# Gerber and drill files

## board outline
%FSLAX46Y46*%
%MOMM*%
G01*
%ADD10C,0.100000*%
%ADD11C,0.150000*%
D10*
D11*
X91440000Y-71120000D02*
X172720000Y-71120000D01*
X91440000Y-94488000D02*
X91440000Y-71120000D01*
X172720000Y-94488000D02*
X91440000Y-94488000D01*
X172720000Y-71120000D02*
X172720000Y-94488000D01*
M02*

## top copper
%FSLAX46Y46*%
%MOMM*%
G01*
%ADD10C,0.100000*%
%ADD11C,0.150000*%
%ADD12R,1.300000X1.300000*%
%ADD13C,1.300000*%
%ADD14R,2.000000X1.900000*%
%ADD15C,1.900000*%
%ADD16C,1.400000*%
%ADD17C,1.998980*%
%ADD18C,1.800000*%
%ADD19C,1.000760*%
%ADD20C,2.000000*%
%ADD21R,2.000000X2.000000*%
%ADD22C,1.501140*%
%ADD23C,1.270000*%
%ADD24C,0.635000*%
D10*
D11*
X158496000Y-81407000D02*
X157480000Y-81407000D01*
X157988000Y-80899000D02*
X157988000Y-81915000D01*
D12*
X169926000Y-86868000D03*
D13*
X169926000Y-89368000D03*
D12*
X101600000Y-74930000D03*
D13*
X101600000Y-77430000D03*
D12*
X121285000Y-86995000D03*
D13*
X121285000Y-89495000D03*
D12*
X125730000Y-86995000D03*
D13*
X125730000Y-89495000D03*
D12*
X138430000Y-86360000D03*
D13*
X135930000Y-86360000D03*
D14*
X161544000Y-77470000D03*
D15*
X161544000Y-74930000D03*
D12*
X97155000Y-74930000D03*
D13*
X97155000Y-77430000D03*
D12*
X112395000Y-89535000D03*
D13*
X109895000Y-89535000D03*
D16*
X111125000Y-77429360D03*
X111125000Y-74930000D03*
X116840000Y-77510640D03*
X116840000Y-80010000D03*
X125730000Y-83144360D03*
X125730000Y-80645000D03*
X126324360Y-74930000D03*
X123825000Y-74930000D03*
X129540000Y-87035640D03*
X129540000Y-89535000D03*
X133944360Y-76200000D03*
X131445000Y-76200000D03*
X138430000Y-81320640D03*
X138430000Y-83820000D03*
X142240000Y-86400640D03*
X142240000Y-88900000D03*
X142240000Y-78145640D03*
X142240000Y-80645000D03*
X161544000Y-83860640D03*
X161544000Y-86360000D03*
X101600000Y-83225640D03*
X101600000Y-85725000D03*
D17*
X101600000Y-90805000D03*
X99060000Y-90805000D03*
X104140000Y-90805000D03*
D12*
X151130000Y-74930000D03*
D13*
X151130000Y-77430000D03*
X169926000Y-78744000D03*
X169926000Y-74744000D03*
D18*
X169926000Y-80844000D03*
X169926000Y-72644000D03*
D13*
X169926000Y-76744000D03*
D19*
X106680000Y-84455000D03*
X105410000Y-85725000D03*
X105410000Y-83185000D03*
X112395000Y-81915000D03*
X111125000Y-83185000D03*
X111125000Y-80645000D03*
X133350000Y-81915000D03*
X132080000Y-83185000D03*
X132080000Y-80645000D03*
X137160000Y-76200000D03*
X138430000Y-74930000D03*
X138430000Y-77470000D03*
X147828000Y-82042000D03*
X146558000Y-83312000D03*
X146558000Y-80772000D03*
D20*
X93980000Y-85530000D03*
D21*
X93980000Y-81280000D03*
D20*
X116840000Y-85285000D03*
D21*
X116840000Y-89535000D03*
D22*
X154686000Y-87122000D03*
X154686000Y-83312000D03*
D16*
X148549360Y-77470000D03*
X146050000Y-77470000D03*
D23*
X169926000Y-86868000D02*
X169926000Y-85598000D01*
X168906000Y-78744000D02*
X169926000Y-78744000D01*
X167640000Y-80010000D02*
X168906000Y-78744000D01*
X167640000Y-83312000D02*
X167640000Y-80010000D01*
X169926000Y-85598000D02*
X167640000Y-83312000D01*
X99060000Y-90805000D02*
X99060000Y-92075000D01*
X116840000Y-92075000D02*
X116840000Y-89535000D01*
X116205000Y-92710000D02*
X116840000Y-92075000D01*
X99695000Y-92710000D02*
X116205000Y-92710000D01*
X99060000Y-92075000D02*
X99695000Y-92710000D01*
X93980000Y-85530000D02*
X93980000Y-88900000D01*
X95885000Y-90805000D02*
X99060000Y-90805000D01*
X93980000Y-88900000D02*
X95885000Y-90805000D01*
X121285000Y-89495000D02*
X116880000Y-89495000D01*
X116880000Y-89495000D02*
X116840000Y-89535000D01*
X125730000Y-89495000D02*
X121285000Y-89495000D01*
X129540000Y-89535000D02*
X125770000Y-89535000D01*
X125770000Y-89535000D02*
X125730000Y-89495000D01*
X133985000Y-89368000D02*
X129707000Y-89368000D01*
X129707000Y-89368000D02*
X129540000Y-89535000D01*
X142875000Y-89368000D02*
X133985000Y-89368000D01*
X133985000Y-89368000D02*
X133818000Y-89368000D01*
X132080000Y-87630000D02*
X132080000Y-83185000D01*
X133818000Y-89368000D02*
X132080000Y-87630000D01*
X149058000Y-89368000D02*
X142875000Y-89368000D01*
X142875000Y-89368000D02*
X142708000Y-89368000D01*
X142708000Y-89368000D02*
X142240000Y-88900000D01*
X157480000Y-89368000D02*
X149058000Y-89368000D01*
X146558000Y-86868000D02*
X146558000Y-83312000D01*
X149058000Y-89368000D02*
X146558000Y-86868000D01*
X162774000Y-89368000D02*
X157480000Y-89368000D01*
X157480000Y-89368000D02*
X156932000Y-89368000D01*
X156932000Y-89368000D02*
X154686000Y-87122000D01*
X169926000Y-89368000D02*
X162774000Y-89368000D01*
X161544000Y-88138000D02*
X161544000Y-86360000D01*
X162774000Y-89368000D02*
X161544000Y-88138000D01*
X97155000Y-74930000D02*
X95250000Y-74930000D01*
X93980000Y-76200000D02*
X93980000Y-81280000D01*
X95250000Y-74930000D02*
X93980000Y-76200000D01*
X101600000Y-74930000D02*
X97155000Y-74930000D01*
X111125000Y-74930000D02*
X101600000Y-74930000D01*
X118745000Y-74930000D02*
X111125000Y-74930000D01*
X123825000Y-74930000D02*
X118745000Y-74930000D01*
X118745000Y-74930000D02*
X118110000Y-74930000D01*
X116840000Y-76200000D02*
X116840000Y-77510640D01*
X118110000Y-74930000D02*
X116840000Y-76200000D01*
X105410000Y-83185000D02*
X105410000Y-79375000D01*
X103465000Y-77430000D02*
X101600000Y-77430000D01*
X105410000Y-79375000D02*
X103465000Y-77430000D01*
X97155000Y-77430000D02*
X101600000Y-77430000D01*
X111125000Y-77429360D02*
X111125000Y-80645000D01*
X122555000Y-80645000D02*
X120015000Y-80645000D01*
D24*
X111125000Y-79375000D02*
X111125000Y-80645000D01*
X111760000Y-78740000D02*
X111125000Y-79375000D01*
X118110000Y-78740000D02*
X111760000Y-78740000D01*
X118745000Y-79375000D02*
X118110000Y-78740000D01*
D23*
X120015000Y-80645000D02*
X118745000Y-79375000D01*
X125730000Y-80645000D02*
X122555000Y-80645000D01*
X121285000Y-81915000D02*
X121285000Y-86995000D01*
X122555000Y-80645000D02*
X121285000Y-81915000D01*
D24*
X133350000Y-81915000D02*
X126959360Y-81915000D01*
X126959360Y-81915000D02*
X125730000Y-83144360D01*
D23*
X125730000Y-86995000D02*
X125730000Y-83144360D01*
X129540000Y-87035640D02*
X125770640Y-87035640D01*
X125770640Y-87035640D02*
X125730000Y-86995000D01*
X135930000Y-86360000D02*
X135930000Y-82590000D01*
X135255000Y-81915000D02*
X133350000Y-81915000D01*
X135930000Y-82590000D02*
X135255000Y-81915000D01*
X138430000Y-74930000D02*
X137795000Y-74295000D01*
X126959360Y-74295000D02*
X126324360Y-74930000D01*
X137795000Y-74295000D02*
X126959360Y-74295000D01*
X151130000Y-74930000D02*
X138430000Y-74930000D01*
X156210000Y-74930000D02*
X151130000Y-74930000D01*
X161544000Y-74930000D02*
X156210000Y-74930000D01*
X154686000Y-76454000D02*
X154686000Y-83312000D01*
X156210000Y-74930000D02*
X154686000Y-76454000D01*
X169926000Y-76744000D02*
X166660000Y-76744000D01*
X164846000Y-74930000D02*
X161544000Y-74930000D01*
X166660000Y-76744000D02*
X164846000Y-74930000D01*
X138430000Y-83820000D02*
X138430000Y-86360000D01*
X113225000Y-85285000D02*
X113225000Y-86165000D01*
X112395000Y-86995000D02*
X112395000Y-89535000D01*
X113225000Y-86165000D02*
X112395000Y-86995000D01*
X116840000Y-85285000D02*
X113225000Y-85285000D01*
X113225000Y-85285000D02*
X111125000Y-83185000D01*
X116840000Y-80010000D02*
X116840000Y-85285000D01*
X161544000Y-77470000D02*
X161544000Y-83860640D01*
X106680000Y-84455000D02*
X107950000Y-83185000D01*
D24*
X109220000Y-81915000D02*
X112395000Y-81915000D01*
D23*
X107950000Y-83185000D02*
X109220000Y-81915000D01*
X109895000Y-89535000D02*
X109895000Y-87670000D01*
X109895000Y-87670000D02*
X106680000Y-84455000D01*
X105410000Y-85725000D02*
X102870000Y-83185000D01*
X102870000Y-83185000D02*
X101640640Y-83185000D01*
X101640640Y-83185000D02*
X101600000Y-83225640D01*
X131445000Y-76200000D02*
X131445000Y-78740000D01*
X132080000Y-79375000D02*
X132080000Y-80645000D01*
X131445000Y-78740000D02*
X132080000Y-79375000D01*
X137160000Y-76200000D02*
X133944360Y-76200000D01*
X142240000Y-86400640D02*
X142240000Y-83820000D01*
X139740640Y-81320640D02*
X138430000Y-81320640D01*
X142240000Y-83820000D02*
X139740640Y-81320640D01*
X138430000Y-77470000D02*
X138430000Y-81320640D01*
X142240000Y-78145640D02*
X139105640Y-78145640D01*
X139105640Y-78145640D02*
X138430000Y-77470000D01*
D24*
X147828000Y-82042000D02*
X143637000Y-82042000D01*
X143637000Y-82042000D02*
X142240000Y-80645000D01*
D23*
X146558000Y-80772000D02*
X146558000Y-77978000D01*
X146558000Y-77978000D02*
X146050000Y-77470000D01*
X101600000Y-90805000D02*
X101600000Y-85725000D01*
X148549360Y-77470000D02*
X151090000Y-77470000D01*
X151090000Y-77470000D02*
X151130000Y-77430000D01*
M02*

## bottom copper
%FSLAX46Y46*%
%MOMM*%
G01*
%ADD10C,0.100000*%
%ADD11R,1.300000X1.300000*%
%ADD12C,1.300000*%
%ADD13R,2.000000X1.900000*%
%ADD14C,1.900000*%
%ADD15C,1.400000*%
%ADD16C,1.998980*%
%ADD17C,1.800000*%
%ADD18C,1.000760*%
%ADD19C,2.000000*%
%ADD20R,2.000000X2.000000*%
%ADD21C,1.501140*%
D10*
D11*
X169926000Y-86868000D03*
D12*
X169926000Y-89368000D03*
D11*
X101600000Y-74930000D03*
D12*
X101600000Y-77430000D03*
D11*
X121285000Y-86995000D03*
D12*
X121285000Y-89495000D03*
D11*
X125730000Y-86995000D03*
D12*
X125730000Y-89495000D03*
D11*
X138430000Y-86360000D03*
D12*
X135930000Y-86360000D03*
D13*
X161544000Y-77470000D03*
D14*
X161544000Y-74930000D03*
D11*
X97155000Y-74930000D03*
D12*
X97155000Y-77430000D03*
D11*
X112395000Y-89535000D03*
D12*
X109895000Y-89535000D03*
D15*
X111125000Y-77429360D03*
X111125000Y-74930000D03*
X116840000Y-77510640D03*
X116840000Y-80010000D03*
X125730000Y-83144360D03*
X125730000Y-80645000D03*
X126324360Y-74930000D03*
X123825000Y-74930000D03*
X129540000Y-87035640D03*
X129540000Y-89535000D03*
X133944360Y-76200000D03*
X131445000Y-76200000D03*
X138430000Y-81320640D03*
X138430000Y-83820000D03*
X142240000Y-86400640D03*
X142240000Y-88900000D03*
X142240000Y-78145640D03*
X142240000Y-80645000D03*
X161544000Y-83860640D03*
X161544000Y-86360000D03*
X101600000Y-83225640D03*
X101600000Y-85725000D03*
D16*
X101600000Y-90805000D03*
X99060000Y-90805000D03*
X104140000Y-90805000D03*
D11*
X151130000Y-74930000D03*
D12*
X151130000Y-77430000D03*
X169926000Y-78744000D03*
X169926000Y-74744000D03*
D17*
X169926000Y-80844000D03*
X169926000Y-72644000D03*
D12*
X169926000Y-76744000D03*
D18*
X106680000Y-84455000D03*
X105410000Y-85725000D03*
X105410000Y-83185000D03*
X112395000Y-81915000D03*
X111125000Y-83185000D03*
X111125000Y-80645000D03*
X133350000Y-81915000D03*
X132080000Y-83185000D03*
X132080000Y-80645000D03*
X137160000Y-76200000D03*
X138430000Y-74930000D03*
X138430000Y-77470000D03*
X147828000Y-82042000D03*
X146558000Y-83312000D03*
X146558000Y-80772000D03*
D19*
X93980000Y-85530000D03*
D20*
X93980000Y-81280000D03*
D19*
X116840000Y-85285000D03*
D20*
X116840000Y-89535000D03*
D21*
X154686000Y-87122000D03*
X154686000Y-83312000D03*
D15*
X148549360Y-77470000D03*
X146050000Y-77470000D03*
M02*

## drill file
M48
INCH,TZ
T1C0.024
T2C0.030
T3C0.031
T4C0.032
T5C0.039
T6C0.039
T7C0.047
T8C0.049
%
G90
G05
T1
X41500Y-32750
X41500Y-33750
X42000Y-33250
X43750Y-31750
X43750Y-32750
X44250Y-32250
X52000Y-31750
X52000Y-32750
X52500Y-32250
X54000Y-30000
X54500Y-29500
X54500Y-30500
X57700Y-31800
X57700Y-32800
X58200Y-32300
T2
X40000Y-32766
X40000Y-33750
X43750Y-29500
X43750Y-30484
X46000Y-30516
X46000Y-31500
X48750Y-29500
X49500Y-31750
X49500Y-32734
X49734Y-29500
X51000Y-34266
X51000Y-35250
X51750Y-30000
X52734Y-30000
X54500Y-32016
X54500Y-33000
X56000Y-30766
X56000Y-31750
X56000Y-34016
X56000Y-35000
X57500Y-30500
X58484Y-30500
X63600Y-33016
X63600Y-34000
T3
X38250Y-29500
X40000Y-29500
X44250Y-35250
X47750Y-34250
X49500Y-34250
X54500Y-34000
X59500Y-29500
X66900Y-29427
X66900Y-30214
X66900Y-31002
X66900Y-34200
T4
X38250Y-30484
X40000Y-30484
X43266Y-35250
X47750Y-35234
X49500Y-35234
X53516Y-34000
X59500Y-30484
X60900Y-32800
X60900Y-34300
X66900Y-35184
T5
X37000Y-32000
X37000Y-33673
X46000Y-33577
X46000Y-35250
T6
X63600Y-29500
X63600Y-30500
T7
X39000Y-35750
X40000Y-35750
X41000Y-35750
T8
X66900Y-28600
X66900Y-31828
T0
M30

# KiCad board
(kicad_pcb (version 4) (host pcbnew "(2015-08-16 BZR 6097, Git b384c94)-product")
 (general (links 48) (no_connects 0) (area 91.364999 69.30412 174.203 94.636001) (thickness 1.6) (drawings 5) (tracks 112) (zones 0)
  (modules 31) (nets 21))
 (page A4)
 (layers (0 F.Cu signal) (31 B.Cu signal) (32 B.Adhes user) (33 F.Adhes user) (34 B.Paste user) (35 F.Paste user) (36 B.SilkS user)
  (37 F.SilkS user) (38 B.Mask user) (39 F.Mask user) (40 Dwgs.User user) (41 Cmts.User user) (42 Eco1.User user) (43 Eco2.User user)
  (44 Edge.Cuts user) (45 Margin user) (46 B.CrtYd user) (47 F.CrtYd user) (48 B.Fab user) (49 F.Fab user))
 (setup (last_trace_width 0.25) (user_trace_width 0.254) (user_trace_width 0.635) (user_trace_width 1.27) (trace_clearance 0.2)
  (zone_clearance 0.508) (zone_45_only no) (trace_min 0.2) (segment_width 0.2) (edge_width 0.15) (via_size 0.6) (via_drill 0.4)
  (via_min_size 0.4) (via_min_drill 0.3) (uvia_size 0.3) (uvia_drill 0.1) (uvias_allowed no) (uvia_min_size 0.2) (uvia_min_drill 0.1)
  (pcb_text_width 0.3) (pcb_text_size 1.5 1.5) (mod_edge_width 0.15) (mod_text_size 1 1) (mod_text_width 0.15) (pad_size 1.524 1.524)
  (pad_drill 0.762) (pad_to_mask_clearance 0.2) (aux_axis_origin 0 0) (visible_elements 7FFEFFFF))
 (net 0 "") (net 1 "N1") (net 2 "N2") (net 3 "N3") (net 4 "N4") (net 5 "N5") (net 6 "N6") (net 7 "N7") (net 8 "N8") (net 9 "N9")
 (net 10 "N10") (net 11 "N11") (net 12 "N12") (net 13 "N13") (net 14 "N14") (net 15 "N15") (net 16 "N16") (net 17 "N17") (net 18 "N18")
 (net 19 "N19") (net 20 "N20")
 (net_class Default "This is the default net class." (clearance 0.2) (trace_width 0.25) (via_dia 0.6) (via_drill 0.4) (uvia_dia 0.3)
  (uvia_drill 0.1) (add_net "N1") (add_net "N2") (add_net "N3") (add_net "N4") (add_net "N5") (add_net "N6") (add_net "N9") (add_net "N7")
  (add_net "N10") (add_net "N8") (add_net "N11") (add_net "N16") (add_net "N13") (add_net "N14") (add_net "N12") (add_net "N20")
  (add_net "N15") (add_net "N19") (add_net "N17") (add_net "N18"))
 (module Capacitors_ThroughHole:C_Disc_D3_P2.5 (layer F.Cu) (at 169.926 86.868 270)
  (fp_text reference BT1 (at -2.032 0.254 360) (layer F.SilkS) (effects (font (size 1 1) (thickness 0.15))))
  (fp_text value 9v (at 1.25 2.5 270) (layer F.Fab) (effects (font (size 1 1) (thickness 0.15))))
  (pad 1 thru_hole rect (at 0 0 270) (size 1.3 1.3) (drill 0.8) (layers *.Cu *.Mask F.SilkS) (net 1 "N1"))
  (pad 2 thru_hole circle (at 2.5 0 270) (size 1.3 1.3) (drill 0.8001) (layers *.Cu *.Mask F.SilkS) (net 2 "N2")))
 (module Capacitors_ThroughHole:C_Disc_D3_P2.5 (layer F.Cu) (at 101.6 74.93 270)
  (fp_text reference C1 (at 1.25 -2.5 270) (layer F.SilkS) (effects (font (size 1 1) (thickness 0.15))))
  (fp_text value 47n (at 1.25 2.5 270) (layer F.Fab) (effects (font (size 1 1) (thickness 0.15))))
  (pad 1 thru_hole rect (at 0 0 270) (size 1.3 1.3) (drill 0.8) (layers *.Cu *.Mask F.SilkS) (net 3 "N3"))
  (pad 2 thru_hole circle (at 2.5 0 270) (size 1.3 1.3) (drill 0.8001) (layers *.Cu *.Mask F.SilkS) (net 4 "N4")))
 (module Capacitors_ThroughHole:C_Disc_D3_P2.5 (layer F.Cu) (at 121.285 86.995 270)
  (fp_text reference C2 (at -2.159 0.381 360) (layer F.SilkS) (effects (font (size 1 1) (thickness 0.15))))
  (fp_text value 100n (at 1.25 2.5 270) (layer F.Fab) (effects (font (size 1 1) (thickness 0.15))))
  (pad 1 thru_hole rect (at 0 0 270) (size 1.3 1.3) (drill 0.8) (layers *.Cu *.Mask F.SilkS) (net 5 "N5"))
  (pad 2 thru_hole circle (at 2.5 0 270) (size 1.3 1.3) (drill 0.8001) (layers *.Cu *.Mask F.SilkS) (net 2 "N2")))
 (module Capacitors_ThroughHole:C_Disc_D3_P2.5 (layer F.Cu) (at 125.73 86.995 270)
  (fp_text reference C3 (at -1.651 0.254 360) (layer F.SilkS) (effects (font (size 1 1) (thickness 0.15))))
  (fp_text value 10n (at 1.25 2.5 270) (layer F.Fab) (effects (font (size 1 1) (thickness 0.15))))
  (pad 1 thru_hole rect (at 0 0 270) (size 1.3 1.3) (drill 0.8) (layers *.Cu *.Mask F.SilkS) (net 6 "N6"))
  (pad 2 thru_hole circle (at 2.5 0 270) (size 1.3 1.3) (drill 0.8001) (layers *.Cu *.Mask F.SilkS) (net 2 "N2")))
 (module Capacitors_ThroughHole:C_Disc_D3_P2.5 (layer F.Cu) (at 138.43 86.36 180)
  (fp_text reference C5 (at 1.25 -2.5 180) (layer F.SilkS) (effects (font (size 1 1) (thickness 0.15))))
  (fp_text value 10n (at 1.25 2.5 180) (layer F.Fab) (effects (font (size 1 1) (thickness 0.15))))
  (pad 1 thru_hole rect (at 0 0 180) (size 1.3 1.3) (drill 0.8) (layers *.Cu *.Mask F.SilkS) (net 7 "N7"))
  (pad 2 thru_hole circle (at 2.5 0 180) (size 1.3 1.3) (drill 0.8001) (layers *.Cu *.Mask F.SilkS) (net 6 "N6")))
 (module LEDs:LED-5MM (layer F.Cu) (at 161.544 77.47 90)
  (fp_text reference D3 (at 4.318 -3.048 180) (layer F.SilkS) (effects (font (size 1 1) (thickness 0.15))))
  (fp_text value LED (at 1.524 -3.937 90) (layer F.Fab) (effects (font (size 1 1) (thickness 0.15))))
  (pad 1 thru_hole rect (at 0 0 180) (size 2 1.9) (drill 1.00076) (layers *.Cu *.Mask F.SilkS) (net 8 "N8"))
  (pad 2 thru_hole circle (at 2.54 0 90) (size 1.9 1.9) (drill 1.00076) (layers *.Cu *.Mask F.SilkS) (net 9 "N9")))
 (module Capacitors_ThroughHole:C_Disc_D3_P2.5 (layer F.Cu) (at 97.155 74.93 270)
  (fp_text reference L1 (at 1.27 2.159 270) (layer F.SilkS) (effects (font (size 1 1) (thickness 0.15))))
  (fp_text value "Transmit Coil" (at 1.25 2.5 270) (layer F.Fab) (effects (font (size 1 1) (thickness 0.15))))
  (pad 1 thru_hole rect (at 0 0 270) (size 1.3 1.3) (drill 0.8) (layers *.Cu *.Mask F.SilkS) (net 3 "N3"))
  (pad 2 thru_hole circle (at 2.5 0 270) (size 1.3 1.3) (drill 0.8001) (layers *.Cu *.Mask F.SilkS) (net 4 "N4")))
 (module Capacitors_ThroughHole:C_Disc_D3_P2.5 (layer F.Cu) (at 112.395 89.535 180)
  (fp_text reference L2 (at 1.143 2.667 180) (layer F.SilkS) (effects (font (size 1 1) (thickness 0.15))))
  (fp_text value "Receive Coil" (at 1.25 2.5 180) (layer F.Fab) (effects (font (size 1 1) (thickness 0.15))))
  (pad 1 thru_hole rect (at 0 0 180) (size 1.3 1.3) (drill 0.8) (layers *.Cu *.Mask F.SilkS) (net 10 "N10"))
  (pad 2 thru_hole circle (at 2.5 0 180) (size 1.3 1.3) (drill 0.8001) (layers *.Cu *.Mask F.SilkS) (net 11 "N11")))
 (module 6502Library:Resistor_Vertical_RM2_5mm (layer F.Cu) (at 111.125 74.93 90)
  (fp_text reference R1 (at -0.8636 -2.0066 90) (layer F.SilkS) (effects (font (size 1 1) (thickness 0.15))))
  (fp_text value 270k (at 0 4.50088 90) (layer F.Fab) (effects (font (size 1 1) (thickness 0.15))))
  (pad 1 thru_hole circle (at -2.49936 0 90) (size 1.4 1.4) (drill 0.76) (layers *.Cu *.SilkS *.Mask) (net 5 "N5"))
  (pad 2 thru_hole circle (at 0 0 90) (size 1.4 1.4) (drill 0.76) (layers *.Cu *.SilkS *.Mask) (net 3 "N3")))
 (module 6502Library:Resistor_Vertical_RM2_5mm (layer F.Cu) (at 116.84 80.01 270)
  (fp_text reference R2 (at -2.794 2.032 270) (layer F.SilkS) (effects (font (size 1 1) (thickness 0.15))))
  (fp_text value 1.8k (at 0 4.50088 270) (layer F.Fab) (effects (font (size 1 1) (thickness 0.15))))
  (pad 1 thru_hole circle (at -2.49936 0 270) (size 1.4 1.4) (drill 0.76) (layers *.Cu *.SilkS *.Mask) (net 3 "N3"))
  (pad 2 thru_hole circle (at 0 0 270) (size 1.4 1.4) (drill 0.76) (layers *.Cu *.SilkS *.Mask) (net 10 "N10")))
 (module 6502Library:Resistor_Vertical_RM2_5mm (layer F.Cu) (at 125.73 80.645 90)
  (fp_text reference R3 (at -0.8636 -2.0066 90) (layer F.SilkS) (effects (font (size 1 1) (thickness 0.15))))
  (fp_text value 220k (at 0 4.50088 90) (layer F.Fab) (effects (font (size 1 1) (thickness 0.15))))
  (pad 1 thru_hole circle (at -2.49936 0 90) (size 1.4 1.4) (drill 0.76) (layers *.Cu *.SilkS *.Mask) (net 6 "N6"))
  (pad 2 thru_hole circle (at 0 0 90) (size 1.4 1.4) (drill 0.76) (layers *.Cu *.SilkS *.Mask) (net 5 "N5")))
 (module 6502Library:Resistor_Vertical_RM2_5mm (layer F.Cu) (at 123.825 74.93 180)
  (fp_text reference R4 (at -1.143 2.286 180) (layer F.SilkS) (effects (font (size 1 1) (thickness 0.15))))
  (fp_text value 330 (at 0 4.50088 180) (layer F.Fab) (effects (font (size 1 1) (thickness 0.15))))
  (pad 1 thru_hole circle (at -2.49936 0 180) (size 1.4 1.4) (drill 0.76) (layers *.Cu *.SilkS *.Mask) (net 9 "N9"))
  (pad 2 thru_hole circle (at 0 0 180) (size 1.4 1.4) (drill 0.76) (layers *.Cu *.SilkS *.Mask) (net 3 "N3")))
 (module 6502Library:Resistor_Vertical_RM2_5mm (layer F.Cu) (at 129.54 89.535 270)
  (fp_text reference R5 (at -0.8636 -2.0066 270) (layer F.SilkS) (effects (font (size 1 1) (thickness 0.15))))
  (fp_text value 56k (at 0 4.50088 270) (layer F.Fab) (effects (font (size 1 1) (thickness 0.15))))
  (pad 1 thru_hole circle (at -2.49936 0 270) (size 1.4 1.4) (drill 0.76) (layers *.Cu *.SilkS *.Mask) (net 6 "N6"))
  (pad 2 thru_hole circle (at 0 0 270) (size 1.4 1.4) (drill 0.76) (layers *.Cu *.SilkS *.Mask) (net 2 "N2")))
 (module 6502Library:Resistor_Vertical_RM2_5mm (layer F.Cu) (at 131.445 76.2 180)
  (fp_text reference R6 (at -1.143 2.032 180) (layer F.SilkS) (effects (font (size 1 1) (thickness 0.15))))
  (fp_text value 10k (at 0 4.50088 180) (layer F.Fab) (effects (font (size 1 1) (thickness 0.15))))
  (pad 1 thru_hole circle (at -2.49936 0 180) (size 1.4 1.4) (drill 0.76) (layers *.Cu *.SilkS *.Mask) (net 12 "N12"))
  (pad 2 thru_hole circle (at 0 0 180) (size 1.4 1.4) (drill 0.76) (layers *.Cu *.SilkS *.Mask) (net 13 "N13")))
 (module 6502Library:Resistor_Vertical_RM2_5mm (layer F.Cu) (at 138.43 83.82 270)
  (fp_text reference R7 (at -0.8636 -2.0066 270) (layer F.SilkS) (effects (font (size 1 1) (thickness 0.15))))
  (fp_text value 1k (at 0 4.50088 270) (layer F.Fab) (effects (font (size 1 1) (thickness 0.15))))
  (pad 1 thru_hole circle (at -2.49936 0 270) (size 1.4 1.4) (drill 0.76) (layers *.Cu *.SilkS *.Mask) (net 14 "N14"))
  (pad 2 thru_hole circle (at 0 0 270) (size 1.4 1.4) (drill 0.76) (layers *.Cu *.SilkS *.Mask) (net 7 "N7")))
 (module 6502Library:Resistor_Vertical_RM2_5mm (layer F.Cu) (at 142.24 88.9 270)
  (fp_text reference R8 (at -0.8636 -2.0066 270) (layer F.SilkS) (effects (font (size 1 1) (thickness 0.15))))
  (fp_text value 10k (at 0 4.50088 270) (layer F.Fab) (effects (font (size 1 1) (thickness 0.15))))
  (pad 1 thru_hole circle (at -2.49936 0 270) (size 1.4 1.4) (drill 0.76) (layers *.Cu *.SilkS *.Mask) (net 14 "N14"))
  (pad 2 thru_hole circle (at 0 0 270) (size 1.4 1.4) (drill 0.76) (layers *.Cu *.SilkS *.Mask) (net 2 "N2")))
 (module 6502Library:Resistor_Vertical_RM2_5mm (layer F.Cu) (at 142.24 80.645 270)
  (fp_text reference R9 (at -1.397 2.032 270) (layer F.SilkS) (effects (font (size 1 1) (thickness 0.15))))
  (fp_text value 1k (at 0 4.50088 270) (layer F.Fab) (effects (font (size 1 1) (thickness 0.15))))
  (pad 1 thru_hole circle (at -2.49936 0 270) (size 1.4 1.4) (drill 0.76) (layers *.Cu *.SilkS *.Mask) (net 14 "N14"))
  (pad 2 thru_hole circle (at 0 0 270) (size 1.4 1.4) (drill 0.76) (layers *.Cu *.SilkS *.Mask) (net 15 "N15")))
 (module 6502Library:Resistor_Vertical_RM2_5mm (layer F.Cu) (at 161.544 86.36 270)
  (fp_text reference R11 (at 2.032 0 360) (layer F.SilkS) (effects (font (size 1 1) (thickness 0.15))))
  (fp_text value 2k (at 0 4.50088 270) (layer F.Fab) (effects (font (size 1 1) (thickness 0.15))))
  (pad 1 thru_hole circle (at -2.49936 0 270) (size 1.4 1.4) (drill 0.76) (layers *.Cu *.SilkS *.Mask) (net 8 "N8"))
  (pad 2 thru_hole circle (at 0 0 270) (size 1.4 1.4) (drill 0.76) (layers *.Cu *.SilkS *.Mask) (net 2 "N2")))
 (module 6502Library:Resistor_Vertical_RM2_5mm (layer F.Cu) (at 101.6 85.725 270)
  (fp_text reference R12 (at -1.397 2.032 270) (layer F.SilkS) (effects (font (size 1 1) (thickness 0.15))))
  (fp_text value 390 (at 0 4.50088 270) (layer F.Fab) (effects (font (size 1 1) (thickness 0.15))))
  (pad 1 thru_hole circle (at -2.49936 0 270) (size 1.4 1.4) (drill 0.76) (layers *.Cu *.SilkS *.Mask) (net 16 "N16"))
  (pad 2 thru_hole circle (at 0 0 270) (size 1.4 1.4) (drill 0.76) (layers *.Cu *.SilkS *.Mask) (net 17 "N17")))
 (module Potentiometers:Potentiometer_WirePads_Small (layer F.Cu) (at 104.14 90.805 270)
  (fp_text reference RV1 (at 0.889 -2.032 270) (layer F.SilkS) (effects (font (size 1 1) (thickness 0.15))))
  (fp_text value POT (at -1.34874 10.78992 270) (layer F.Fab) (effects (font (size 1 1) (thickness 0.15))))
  (pad 2 thru_hole circle (at 0 2.54 270) (size 1.99898 1.99898) (drill 1.19888) (layers *.Cu *.Mask F.SilkS) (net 17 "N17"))
  (pad 3 thru_hole circle (at 0 5.08 270) (size 1.99898 1.99898) (drill 1.19888) (layers *.Cu *.Mask F.SilkS) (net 2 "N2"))
  (pad 1 thru_hole circle (at 0 0 270) (size 1.99898 1.99898) (drill 1.19888) (layers *.Cu *.Mask F.SilkS) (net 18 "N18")))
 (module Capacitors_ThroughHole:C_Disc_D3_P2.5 (layer F.Cu) (at 151.13 74.93 270)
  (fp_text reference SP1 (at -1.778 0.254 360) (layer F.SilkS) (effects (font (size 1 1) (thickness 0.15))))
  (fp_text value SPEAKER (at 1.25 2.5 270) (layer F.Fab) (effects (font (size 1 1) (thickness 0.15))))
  (pad 1 thru_hole rect (at 0 0 270) (size 1.3 1.3) (drill 0.8) (layers *.Cu *.Mask F.SilkS) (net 9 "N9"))
  (pad 2 thru_hole circle (at 2.5 0 270) (size 1.3 1.3) (drill 0.8001) (layers *.Cu *.Mask F.SilkS) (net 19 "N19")))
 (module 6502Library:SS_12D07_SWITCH (layer F.Cu) (at 169.926 72.644 270)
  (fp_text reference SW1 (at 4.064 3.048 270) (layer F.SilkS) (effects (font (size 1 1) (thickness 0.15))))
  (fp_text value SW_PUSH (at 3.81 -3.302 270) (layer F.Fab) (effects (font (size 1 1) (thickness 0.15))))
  (pad 2 thru_hole circle (at 6.1 0 270) (size 1.3 1.3) (drill 0.8) (layers *.Cu *.Mask F.SilkS) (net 1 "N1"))
  (pad "" thru_hole circle (at 2.1 0 270) (size 1.3 1.3) (drill 0.8) (layers *.Cu *.Mask F.SilkS))
  (pad "" thru_hole circle (at 8.2 0 270) (size 1.8 1.8) (drill 1.25) (layers *.Cu *.Mask F.SilkS))
  (pad "" thru_hole circle (at 0 0 270) (size 1.8 1.8) (drill 1.25) (layers *.Cu *.Mask F.SilkS))
  (pad 1 thru_hole circle (at 4.1 0 270) (size 1.3 1.3) (drill 0.8) (layers *.Cu *.Mask F.SilkS) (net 9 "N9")))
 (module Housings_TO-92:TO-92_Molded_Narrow (layer F.Cu) (at 105.41 83.185 270)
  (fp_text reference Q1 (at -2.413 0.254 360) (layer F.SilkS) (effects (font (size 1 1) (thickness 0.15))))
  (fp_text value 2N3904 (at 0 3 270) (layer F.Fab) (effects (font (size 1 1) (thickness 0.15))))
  (pad 2 thru_hole circle (at 1.27 -1.27) (size 1.00076 1.00076) (drill 0.6) (layers *.Cu *.Mask F.SilkS) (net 11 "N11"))
  (pad 3 thru_hole circle (at 2.54 0) (size 1.00076 1.00076) (drill 0.6) (layers *.Cu *.Mask F.SilkS) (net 16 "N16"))
  (pad 1 thru_hole circle (at 0 0) (size 1.00076 1.00076) (drill 0.6) (layers *.Cu *.Mask F.SilkS) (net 4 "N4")))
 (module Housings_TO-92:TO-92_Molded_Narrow (layer F.Cu) (at 111.125 80.645 270)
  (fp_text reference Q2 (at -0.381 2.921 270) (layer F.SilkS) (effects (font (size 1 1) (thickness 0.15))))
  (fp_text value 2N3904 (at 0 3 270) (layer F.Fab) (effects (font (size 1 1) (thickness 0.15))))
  (pad 2 thru_hole circle (at 1.27 -1.27) (size 1.00076 1.00076) (drill 0.6) (layers *.Cu *.Mask F.SilkS) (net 11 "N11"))
  (pad 3 thru_hole circle (at 2.54 0) (size 1.00076 1.00076) (drill 0.6) (layers *.Cu *.Mask F.SilkS) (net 10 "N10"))
  (pad 1 thru_hole circle (at 0 0) (size 1.00076 1.00076) (drill 0.6) (layers *.Cu *.Mask F.SilkS) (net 5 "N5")))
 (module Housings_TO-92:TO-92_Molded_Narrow (layer F.Cu) (at 132.08 80.645 270)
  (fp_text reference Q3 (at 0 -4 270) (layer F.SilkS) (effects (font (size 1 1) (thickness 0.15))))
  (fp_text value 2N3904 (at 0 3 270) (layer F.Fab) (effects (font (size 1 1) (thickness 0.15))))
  (pad 2 thru_hole circle (at 1.27 -1.27) (size 1.00076 1.00076) (drill 0.6) (layers *.Cu *.Mask F.SilkS) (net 6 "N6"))
  (pad 3 thru_hole circle (at 2.54 0) (size 1.00076 1.00076) (drill 0.6) (layers *.Cu *.Mask F.SilkS) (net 2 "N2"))
  (pad 1 thru_hole circle (at 0 0) (size 1.00076 1.00076) (drill 0.6) (layers *.Cu *.Mask F.SilkS) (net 13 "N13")))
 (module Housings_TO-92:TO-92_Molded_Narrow (layer F.Cu) (at 138.43 77.47 90)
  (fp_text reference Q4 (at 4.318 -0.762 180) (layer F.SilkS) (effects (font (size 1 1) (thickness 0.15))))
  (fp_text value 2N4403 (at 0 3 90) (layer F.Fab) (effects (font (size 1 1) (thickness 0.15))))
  (pad 2 thru_hole circle (at 1.27 -1.27 180) (size 1.00076 1.00076) (drill 0.6) (layers *.Cu *.Mask F.SilkS) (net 12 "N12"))
  (pad 3 thru_hole circle (at 2.54 0 180) (size 1.00076 1.00076) (drill 0.6) (layers *.Cu *.Mask F.SilkS) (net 9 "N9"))
  (pad 1 thru_hole circle (at 0 0 180) (size 1.00076 1.00076) (drill 0.6) (layers *.Cu *.Mask F.SilkS) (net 14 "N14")))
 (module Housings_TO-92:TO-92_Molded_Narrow (layer F.Cu) (at 146.558 80.772 270)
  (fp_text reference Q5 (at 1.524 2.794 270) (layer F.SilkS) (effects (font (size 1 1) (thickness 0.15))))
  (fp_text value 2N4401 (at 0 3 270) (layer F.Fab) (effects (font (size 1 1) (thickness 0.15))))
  (pad 2 thru_hole circle (at 1.27 -1.27) (size 1.00076 1.00076) (drill 0.6) (layers *.Cu *.Mask F.SilkS) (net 15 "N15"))
  (pad 3 thru_hole circle (at 2.54 0) (size 1.00076 1.00076) (drill 0.6) (layers *.Cu *.Mask F.SilkS) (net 2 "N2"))
  (pad 1 thru_hole circle (at 0 0) (size 1.00076 1.00076) (drill 0.6) (layers *.Cu *.Mask F.SilkS) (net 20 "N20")))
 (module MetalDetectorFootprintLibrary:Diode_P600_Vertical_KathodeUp (layer F.Cu) (at 93.98 81.28 270)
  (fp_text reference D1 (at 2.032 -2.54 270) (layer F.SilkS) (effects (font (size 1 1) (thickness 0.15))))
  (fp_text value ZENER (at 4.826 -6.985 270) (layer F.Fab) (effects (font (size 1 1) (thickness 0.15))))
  (pad 2 thru_hole circle (at 4.25 0 90) (size 2 2) (drill 1) (layers *.Cu *.Mask F.SilkS) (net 2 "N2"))
  (pad 1 thru_hole rect (at 0 0 90) (size 2 2) (drill 1) (layers *.Cu *.Mask F.SilkS) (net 3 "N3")))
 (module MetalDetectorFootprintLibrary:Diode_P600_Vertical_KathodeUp (layer F.Cu) (at 116.84 89.535 90)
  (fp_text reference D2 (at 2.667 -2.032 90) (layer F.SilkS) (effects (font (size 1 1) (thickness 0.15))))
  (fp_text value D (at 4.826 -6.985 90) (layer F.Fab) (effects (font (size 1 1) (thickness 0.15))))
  (pad 2 thru_hole circle (at 4.25 0 270) (size 2 2) (drill 1) (layers *.Cu *.Mask F.SilkS) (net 10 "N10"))
  (pad 1 thru_hole rect (at 0 0 270) (size 2 2) (drill 1) (layers *.Cu *.Mask F.SilkS) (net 2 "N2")))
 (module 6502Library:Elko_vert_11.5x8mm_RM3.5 (layer F.Cu) (at 154.686 83.312 270)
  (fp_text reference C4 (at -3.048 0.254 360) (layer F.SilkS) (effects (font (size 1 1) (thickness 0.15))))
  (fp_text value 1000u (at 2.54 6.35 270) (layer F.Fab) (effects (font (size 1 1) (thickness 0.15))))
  (fp_line (start -1.905 -3.81) (end -1.905 -2.794) (layer F.Cu) (width 0.15))
  (fp_line (start -2.413 -3.302) (end -1.397 -3.302) (layer F.Cu) (width 0.15))
  (pad 2 thru_hole circle (at 3.81 0 270) (size 1.50114 1.50114) (drill 0.8001) (layers *.Cu *.Mask F.SilkS) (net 2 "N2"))
  (pad 1 thru_hole circle (at 0 0 270) (size 1.50114 1.50114) (drill 0.8001) (layers *.Cu *.Mask F.SilkS) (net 9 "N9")))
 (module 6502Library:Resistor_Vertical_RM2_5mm (layer F.Cu) (at 146.05 77.47 180)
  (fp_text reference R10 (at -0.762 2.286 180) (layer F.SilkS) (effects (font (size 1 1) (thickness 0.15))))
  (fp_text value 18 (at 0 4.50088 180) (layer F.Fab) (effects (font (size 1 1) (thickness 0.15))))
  (pad 1 thru_hole circle (at -2.49936 0 180) (size 1.4 1.4) (drill 0.76) (layers *.Cu *.SilkS *.Mask) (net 19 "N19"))
  (pad 2 thru_hole circle (at 0 0 180) (size 1.4 1.4) (drill 0.76) (layers *.Cu *.SilkS *.Mask) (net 20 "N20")))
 (gr_line (start 91.44 71.12) (end 172.72 71.12) (angle 90) (layer Edge.Cuts) (width 0.15))
 (gr_line (start 91.44 94.488) (end 91.44 71.12) (angle 90) (layer Edge.Cuts) (width 0.15))
 (gr_line (start 172.72 94.488) (end 91.44 94.488) (angle 90) (layer Edge.Cuts) (width 0.15))
 (gr_line (start 172.72 71.12) (end 172.72 94.488) (angle 90) (layer Edge.Cuts) (width 0.15))
 (segment (start 169.926 86.868) (end 169.926 85.598) (width 1.27) (layer F.Cu) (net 1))
 (segment (start 168.906 78.744) (end 169.926 78.744) (width 1.27) (layer F.Cu) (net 1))
 (segment (start 167.64 80.01) (end 168.906 78.744) (width 1.27) (layer F.Cu) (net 1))
 (segment (start 167.64 83.312) (end 167.64 80.01) (width 1.27) (layer F.Cu) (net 1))
 (segment (start 169.926 85.598) (end 167.64 83.312) (width 1.27) (layer F.Cu) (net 1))
 (segment (start 99.06 90.805) (end 99.06 92.075) (width 1.27) (layer F.Cu) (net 2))
 (segment (start 116.84 92.075) (end 116.84 89.535) (width 1.27) (layer F.Cu) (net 2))
 (segment (start 116.205 92.71) (end 116.84 92.075) (width 1.27) (layer F.Cu) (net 2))
 (segment (start 99.695 92.71) (end 116.205 92.71) (width 1.27) (layer F.Cu) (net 2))
 (segment (start 99.06 92.075) (end 99.695 92.71) (width 1.27) (layer F.Cu) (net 2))
 (segment (start 93.98 85.53) (end 93.98 88.9) (width 1.27) (layer F.Cu) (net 2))
 (segment (start 95.885 90.805) (end 99.06 90.805) (width 1.27) (layer F.Cu) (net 2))
 (segment (start 93.98 88.9) (end 95.885 90.805) (width 1.27) (layer F.Cu) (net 2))
 (segment (start 121.285 89.495) (end 116.88 89.495) (width 1.27) (layer F.Cu) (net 2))
 (segment (start 116.88 89.495) (end 116.84 89.535) (width 1.27) (layer F.Cu) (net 2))
 (segment (start 125.73 89.495) (end 121.285 89.495) (width 1.27) (layer F.Cu) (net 2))
 (segment (start 129.54 89.535) (end 125.77 89.535) (width 1.27) (layer F.Cu) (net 2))
 (segment (start 125.77 89.535) (end 125.73 89.495) (width 1.27) (layer F.Cu) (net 2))
 (segment (start 133.985 89.368) (end 129.707 89.368) (width 1.27) (layer F.Cu) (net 2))
 (segment (start 129.707 89.368) (end 129.54 89.535) (width 1.27) (layer F.Cu) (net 2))
 (segment (start 142.875 89.368) (end 133.985 89.368) (width 1.27) (layer F.Cu) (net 2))
 (segment (start 133.985 89.368) (end 133.818 89.368) (width 1.27) (layer F.Cu) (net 2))
 (segment (start 132.08 87.63) (end 132.08 83.185) (width 1.27) (layer F.Cu) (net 2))
 (segment (start 133.818 89.368) (end 132.08 87.63) (width 1.27) (layer F.Cu) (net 2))
 (segment (start 149.058 89.368) (end 142.875 89.368) (width 1.27) (layer F.Cu) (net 2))
 (segment (start 142.875 89.368) (end 142.708 89.368) (width 1.27) (layer F.Cu) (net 2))
 (segment (start 142.708 89.368) (end 142.24 88.9) (width 1.27) (layer F.Cu) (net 2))
 (segment (start 157.48 89.368) (end 149.058 89.368) (width 1.27) (layer F.Cu) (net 2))
 (segment (start 146.558 86.868) (end 146.558 83.312) (width 1.27) (layer F.Cu) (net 2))
 (segment (start 149.058 89.368) (end 146.558 86.868) (width 1.27) (layer F.Cu) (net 2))
 (segment (start 162.774 89.368) (end 157.48 89.368) (width 1.27) (layer F.Cu) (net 2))
 (segment (start 157.48 89.368) (end 156.932 89.368) (width 1.27) (layer F.Cu) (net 2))
 (segment (start 156.932 89.368) (end 154.686 87.122) (width 1.27) (layer F.Cu) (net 2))
 (segment (start 169.926 89.368) (end 162.774 89.368) (width 1.27) (layer F.Cu) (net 2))
 (segment (start 161.544 88.138) (end 161.544 86.36) (width 1.27) (layer F.Cu) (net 2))
 (segment (start 162.774 89.368) (end 161.544 88.138) (width 1.27) (layer F.Cu) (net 2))
 (segment (start 97.155 74.93) (end 95.25 74.93) (width 1.27) (layer F.Cu) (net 3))
 (segment (start 93.98 76.2) (end 93.98 81.28) (width 1.27) (layer F.Cu) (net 3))
 (segment (start 95.25 74.93) (end 93.98 76.2) (width 1.27) (layer F.Cu) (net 3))
 (segment (start 101.6 74.93) (end 97.155 74.93) (width 1.27) (layer F.Cu) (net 3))
 (segment (start 111.125 74.93) (end 101.6 74.93) (width 1.27) (layer F.Cu) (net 3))
 (segment (start 118.745 74.93) (end 111.125 74.93) (width 1.27) (layer F.Cu) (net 3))
 (segment (start 123.825 74.93) (end 118.745 74.93) (width 1.27) (layer F.Cu) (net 3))
 (segment (start 118.745 74.93) (end 118.11 74.93) (width 1.27) (layer F.Cu) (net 3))
 (segment (start 116.84 76.2) (end 116.84 77.51064) (width 1.27) (layer F.Cu) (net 3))
 (segment (start 118.11 74.93) (end 116.84 76.2) (width 1.27) (layer F.Cu) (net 3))
 (segment (start 105.41 83.185) (end 105.41 79.375) (width 1.27) (layer F.Cu) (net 4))
 (segment (start 103.465 77.43) (end 101.6 77.43) (width 1.27) (layer F.Cu) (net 4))
 (segment (start 105.41 79.375) (end 103.465 77.43) (width 1.27) (layer F.Cu) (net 4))
 (segment (start 97.155 77.43) (end 101.6 77.43) (width 1.27) (layer F.Cu) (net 4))
 (segment (start 111.125 77.42936) (end 111.125 80.645) (width 1.27) (layer F.Cu) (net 5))
 (segment (start 122.555 80.645) (end 120.015 80.645) (width 1.27) (layer F.Cu) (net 5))
 (segment (start 111.125 79.375) (end 111.125 80.645) (width 0.635) (layer F.Cu) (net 5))
 (segment (start 111.76 78.74) (end 111.125 79.375) (width 0.635) (layer F.Cu) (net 5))
 (segment (start 118.11 78.74) (end 111.76 78.74) (width 0.635) (layer F.Cu) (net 5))
 (segment (start 118.745 79.375) (end 118.11 78.74) (width 0.635) (layer F.Cu) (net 5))
 (segment (start 120.015 80.645) (end 118.745 79.375) (width 1.27) (layer F.Cu) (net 5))
 (segment (start 125.73 80.645) (end 122.555 80.645) (width 1.27) (layer F.Cu) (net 5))
 (segment (start 121.285 81.915) (end 121.285 86.995) (width 1.27) (layer F.Cu) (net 5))
 (segment (start 122.555 80.645) (end 121.285 81.915) (width 1.27) (layer F.Cu) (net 5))
 (segment (start 133.35 81.915) (end 126.95936 81.915) (width 0.635) (layer F.Cu) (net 6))
 (segment (start 126.95936 81.915) (end 125.73 83.14436) (width 0.635) (layer F.Cu) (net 6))
 (segment (start 125.73 86.995) (end 125.73 83.14436) (width 1.27) (layer F.Cu) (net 6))
 (segment (start 129.54 87.03564) (end 125.77064 87.03564) (width 1.27) (layer F.Cu) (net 6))
 (segment (start 125.77064 87.03564) (end 125.73 86.995) (width 1.27) (layer F.Cu) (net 6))
 (segment (start 135.93 86.36) (end 135.93 82.59) (width 1.27) (layer F.Cu) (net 6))
 (segment (start 135.255 81.915) (end 133.35 81.915) (width 1.27) (layer F.Cu) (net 6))
 (segment (start 135.93 82.59) (end 135.255 81.915) (width 1.27) (layer F.Cu) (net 6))
 (segment (start 138.43 74.93) (end 137.795 74.295) (width 1.27) (layer F.Cu) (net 9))
 (segment (start 126.95936 74.295) (end 126.32436 74.93) (width 1.27) (layer F.Cu) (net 9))
 (segment (start 137.795 74.295) (end 126.95936 74.295) (width 1.27) (layer F.Cu) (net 9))
 (segment (start 151.13 74.93) (end 138.43 74.93) (width 1.27) (layer F.Cu) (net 9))
 (segment (start 156.21 74.93) (end 151.13 74.93) (width 1.27) (layer F.Cu) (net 9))
 (segment (start 161.544 74.93) (end 156.21 74.93) (width 1.27) (layer F.Cu) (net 9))
 (segment (start 154.686 76.454) (end 154.686 83.312) (width 1.27) (layer F.Cu) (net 9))
 (segment (start 156.21 74.93) (end 154.686 76.454) (width 1.27) (layer F.Cu) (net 9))
 (segment (start 169.926 76.744) (end 166.66 76.744) (width 1.27) (layer F.Cu) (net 9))
 (segment (start 164.846 74.93) (end 161.544 74.93) (width 1.27) (layer F.Cu) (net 9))
 (segment (start 166.66 76.744) (end 164.846 74.93) (width 1.27) (layer F.Cu) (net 9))
 (segment (start 138.43 83.82) (end 138.43 86.36) (width 1.27) (layer F.Cu) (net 7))
 (segment (start 113.225 85.285) (end 113.225 86.165) (width 1.27) (layer F.Cu) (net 10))
 (segment (start 112.395 86.995) (end 112.395 89.535) (width 1.27) (layer F.Cu) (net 10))
 (segment (start 113.225 86.165) (end 112.395 86.995) (width 1.27) (layer F.Cu) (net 10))
 (segment (start 116.84 85.285) (end 113.225 85.285) (width 1.27) (layer F.Cu) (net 10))
 (segment (start 113.225 85.285) (end 111.125 83.185) (width 1.27) (layer F.Cu) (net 10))
 (segment (start 116.84 80.01) (end 116.84 85.285) (width 1.27) (layer F.Cu) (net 10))
 (segment (start 161.544 77.47) (end 161.544 83.86064) (width 1.27) (layer F.Cu) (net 8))
 (segment (start 106.68 84.455) (end 107.95 83.185) (width 1.27) (layer F.Cu) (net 11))
 (segment (start 109.22 81.915) (end 112.395 81.915) (width 0.635) (layer F.Cu) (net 11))
 (segment (start 107.95 83.185) (end 109.22 81.915) (width 1.27) (layer F.Cu) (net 11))
 (segment (start 109.895 89.535) (end 109.895 87.67) (width 1.27) (layer F.Cu) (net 11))
 (segment (start 109.895 87.67) (end 106.68 84.455) (width 1.27) (layer F.Cu) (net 11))
 (segment (start 105.41 85.725) (end 102.87 83.185) (width 1.27) (layer F.Cu) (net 16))
 (segment (start 102.87 83.185) (end 101.64064 83.185) (width 1.27) (layer F.Cu) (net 16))
 (segment (start 101.64064 83.185) (end 101.6 83.22564) (width 1.27) (layer F.Cu) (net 16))
 (segment (start 131.445 76.2) (end 131.445 78.74) (width 1.27) (layer F.Cu) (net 13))
 (segment (start 132.08 79.375) (end 132.08 80.645) (width 1.27) (layer F.Cu) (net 13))
 (segment (start 131.445 78.74) (end 132.08 79.375) (width 1.27) (layer F.Cu) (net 13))
 (segment (start 137.16 76.2) (end 133.94436 76.2) (width 1.27) (layer F.Cu) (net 12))
 (segment (start 142.24 86.40064) (end 142.24 83.82) (width 1.27) (layer F.Cu) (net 14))
 (segment (start 139.74064 81.32064) (end 138.43 81.32064) (width 1.27) (layer F.Cu) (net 14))
 (segment (start 142.24 83.82) (end 139.74064 81.32064) (width 1.27) (layer F.Cu) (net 14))
 (segment (start 138.43 77.47) (end 138.43 81.32064) (width 1.27) (layer F.Cu) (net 14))
 (segment (start 142.24 78.14564) (end 139.10564 78.14564) (width 1.27) (layer F.Cu) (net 14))
 (segment (start 139.10564 78.14564) (end 138.43 77.47) (width 1.27) (layer F.Cu) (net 14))
 (segment (start 147.828 82.042) (end 143.637 82.042) (width 0.635) (layer F.Cu) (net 15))
 (segment (start 143.637 82.042) (end 142.24 80.645) (width 0.635) (layer F.Cu) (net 15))
 (segment (start 146.558 80.772) (end 146.558 77.978) (width 1.27) (layer F.Cu) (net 20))
 (segment (start 146.558 77.978) (end 146.05 77.47) (width 1.27) (layer F.Cu) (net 20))
 (segment (start 101.6 90.805) (end 101.6 85.725) (width 1.27) (layer F.Cu) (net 17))
 (segment (start 148.54936 77.47) (end 151.09 77.47) (width 1.27) (layer F.Cu) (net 19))
 (segment (start 151.09 77.47) (end 151.13 77.43) (width 1.27) (layer F.Cu) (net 19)))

